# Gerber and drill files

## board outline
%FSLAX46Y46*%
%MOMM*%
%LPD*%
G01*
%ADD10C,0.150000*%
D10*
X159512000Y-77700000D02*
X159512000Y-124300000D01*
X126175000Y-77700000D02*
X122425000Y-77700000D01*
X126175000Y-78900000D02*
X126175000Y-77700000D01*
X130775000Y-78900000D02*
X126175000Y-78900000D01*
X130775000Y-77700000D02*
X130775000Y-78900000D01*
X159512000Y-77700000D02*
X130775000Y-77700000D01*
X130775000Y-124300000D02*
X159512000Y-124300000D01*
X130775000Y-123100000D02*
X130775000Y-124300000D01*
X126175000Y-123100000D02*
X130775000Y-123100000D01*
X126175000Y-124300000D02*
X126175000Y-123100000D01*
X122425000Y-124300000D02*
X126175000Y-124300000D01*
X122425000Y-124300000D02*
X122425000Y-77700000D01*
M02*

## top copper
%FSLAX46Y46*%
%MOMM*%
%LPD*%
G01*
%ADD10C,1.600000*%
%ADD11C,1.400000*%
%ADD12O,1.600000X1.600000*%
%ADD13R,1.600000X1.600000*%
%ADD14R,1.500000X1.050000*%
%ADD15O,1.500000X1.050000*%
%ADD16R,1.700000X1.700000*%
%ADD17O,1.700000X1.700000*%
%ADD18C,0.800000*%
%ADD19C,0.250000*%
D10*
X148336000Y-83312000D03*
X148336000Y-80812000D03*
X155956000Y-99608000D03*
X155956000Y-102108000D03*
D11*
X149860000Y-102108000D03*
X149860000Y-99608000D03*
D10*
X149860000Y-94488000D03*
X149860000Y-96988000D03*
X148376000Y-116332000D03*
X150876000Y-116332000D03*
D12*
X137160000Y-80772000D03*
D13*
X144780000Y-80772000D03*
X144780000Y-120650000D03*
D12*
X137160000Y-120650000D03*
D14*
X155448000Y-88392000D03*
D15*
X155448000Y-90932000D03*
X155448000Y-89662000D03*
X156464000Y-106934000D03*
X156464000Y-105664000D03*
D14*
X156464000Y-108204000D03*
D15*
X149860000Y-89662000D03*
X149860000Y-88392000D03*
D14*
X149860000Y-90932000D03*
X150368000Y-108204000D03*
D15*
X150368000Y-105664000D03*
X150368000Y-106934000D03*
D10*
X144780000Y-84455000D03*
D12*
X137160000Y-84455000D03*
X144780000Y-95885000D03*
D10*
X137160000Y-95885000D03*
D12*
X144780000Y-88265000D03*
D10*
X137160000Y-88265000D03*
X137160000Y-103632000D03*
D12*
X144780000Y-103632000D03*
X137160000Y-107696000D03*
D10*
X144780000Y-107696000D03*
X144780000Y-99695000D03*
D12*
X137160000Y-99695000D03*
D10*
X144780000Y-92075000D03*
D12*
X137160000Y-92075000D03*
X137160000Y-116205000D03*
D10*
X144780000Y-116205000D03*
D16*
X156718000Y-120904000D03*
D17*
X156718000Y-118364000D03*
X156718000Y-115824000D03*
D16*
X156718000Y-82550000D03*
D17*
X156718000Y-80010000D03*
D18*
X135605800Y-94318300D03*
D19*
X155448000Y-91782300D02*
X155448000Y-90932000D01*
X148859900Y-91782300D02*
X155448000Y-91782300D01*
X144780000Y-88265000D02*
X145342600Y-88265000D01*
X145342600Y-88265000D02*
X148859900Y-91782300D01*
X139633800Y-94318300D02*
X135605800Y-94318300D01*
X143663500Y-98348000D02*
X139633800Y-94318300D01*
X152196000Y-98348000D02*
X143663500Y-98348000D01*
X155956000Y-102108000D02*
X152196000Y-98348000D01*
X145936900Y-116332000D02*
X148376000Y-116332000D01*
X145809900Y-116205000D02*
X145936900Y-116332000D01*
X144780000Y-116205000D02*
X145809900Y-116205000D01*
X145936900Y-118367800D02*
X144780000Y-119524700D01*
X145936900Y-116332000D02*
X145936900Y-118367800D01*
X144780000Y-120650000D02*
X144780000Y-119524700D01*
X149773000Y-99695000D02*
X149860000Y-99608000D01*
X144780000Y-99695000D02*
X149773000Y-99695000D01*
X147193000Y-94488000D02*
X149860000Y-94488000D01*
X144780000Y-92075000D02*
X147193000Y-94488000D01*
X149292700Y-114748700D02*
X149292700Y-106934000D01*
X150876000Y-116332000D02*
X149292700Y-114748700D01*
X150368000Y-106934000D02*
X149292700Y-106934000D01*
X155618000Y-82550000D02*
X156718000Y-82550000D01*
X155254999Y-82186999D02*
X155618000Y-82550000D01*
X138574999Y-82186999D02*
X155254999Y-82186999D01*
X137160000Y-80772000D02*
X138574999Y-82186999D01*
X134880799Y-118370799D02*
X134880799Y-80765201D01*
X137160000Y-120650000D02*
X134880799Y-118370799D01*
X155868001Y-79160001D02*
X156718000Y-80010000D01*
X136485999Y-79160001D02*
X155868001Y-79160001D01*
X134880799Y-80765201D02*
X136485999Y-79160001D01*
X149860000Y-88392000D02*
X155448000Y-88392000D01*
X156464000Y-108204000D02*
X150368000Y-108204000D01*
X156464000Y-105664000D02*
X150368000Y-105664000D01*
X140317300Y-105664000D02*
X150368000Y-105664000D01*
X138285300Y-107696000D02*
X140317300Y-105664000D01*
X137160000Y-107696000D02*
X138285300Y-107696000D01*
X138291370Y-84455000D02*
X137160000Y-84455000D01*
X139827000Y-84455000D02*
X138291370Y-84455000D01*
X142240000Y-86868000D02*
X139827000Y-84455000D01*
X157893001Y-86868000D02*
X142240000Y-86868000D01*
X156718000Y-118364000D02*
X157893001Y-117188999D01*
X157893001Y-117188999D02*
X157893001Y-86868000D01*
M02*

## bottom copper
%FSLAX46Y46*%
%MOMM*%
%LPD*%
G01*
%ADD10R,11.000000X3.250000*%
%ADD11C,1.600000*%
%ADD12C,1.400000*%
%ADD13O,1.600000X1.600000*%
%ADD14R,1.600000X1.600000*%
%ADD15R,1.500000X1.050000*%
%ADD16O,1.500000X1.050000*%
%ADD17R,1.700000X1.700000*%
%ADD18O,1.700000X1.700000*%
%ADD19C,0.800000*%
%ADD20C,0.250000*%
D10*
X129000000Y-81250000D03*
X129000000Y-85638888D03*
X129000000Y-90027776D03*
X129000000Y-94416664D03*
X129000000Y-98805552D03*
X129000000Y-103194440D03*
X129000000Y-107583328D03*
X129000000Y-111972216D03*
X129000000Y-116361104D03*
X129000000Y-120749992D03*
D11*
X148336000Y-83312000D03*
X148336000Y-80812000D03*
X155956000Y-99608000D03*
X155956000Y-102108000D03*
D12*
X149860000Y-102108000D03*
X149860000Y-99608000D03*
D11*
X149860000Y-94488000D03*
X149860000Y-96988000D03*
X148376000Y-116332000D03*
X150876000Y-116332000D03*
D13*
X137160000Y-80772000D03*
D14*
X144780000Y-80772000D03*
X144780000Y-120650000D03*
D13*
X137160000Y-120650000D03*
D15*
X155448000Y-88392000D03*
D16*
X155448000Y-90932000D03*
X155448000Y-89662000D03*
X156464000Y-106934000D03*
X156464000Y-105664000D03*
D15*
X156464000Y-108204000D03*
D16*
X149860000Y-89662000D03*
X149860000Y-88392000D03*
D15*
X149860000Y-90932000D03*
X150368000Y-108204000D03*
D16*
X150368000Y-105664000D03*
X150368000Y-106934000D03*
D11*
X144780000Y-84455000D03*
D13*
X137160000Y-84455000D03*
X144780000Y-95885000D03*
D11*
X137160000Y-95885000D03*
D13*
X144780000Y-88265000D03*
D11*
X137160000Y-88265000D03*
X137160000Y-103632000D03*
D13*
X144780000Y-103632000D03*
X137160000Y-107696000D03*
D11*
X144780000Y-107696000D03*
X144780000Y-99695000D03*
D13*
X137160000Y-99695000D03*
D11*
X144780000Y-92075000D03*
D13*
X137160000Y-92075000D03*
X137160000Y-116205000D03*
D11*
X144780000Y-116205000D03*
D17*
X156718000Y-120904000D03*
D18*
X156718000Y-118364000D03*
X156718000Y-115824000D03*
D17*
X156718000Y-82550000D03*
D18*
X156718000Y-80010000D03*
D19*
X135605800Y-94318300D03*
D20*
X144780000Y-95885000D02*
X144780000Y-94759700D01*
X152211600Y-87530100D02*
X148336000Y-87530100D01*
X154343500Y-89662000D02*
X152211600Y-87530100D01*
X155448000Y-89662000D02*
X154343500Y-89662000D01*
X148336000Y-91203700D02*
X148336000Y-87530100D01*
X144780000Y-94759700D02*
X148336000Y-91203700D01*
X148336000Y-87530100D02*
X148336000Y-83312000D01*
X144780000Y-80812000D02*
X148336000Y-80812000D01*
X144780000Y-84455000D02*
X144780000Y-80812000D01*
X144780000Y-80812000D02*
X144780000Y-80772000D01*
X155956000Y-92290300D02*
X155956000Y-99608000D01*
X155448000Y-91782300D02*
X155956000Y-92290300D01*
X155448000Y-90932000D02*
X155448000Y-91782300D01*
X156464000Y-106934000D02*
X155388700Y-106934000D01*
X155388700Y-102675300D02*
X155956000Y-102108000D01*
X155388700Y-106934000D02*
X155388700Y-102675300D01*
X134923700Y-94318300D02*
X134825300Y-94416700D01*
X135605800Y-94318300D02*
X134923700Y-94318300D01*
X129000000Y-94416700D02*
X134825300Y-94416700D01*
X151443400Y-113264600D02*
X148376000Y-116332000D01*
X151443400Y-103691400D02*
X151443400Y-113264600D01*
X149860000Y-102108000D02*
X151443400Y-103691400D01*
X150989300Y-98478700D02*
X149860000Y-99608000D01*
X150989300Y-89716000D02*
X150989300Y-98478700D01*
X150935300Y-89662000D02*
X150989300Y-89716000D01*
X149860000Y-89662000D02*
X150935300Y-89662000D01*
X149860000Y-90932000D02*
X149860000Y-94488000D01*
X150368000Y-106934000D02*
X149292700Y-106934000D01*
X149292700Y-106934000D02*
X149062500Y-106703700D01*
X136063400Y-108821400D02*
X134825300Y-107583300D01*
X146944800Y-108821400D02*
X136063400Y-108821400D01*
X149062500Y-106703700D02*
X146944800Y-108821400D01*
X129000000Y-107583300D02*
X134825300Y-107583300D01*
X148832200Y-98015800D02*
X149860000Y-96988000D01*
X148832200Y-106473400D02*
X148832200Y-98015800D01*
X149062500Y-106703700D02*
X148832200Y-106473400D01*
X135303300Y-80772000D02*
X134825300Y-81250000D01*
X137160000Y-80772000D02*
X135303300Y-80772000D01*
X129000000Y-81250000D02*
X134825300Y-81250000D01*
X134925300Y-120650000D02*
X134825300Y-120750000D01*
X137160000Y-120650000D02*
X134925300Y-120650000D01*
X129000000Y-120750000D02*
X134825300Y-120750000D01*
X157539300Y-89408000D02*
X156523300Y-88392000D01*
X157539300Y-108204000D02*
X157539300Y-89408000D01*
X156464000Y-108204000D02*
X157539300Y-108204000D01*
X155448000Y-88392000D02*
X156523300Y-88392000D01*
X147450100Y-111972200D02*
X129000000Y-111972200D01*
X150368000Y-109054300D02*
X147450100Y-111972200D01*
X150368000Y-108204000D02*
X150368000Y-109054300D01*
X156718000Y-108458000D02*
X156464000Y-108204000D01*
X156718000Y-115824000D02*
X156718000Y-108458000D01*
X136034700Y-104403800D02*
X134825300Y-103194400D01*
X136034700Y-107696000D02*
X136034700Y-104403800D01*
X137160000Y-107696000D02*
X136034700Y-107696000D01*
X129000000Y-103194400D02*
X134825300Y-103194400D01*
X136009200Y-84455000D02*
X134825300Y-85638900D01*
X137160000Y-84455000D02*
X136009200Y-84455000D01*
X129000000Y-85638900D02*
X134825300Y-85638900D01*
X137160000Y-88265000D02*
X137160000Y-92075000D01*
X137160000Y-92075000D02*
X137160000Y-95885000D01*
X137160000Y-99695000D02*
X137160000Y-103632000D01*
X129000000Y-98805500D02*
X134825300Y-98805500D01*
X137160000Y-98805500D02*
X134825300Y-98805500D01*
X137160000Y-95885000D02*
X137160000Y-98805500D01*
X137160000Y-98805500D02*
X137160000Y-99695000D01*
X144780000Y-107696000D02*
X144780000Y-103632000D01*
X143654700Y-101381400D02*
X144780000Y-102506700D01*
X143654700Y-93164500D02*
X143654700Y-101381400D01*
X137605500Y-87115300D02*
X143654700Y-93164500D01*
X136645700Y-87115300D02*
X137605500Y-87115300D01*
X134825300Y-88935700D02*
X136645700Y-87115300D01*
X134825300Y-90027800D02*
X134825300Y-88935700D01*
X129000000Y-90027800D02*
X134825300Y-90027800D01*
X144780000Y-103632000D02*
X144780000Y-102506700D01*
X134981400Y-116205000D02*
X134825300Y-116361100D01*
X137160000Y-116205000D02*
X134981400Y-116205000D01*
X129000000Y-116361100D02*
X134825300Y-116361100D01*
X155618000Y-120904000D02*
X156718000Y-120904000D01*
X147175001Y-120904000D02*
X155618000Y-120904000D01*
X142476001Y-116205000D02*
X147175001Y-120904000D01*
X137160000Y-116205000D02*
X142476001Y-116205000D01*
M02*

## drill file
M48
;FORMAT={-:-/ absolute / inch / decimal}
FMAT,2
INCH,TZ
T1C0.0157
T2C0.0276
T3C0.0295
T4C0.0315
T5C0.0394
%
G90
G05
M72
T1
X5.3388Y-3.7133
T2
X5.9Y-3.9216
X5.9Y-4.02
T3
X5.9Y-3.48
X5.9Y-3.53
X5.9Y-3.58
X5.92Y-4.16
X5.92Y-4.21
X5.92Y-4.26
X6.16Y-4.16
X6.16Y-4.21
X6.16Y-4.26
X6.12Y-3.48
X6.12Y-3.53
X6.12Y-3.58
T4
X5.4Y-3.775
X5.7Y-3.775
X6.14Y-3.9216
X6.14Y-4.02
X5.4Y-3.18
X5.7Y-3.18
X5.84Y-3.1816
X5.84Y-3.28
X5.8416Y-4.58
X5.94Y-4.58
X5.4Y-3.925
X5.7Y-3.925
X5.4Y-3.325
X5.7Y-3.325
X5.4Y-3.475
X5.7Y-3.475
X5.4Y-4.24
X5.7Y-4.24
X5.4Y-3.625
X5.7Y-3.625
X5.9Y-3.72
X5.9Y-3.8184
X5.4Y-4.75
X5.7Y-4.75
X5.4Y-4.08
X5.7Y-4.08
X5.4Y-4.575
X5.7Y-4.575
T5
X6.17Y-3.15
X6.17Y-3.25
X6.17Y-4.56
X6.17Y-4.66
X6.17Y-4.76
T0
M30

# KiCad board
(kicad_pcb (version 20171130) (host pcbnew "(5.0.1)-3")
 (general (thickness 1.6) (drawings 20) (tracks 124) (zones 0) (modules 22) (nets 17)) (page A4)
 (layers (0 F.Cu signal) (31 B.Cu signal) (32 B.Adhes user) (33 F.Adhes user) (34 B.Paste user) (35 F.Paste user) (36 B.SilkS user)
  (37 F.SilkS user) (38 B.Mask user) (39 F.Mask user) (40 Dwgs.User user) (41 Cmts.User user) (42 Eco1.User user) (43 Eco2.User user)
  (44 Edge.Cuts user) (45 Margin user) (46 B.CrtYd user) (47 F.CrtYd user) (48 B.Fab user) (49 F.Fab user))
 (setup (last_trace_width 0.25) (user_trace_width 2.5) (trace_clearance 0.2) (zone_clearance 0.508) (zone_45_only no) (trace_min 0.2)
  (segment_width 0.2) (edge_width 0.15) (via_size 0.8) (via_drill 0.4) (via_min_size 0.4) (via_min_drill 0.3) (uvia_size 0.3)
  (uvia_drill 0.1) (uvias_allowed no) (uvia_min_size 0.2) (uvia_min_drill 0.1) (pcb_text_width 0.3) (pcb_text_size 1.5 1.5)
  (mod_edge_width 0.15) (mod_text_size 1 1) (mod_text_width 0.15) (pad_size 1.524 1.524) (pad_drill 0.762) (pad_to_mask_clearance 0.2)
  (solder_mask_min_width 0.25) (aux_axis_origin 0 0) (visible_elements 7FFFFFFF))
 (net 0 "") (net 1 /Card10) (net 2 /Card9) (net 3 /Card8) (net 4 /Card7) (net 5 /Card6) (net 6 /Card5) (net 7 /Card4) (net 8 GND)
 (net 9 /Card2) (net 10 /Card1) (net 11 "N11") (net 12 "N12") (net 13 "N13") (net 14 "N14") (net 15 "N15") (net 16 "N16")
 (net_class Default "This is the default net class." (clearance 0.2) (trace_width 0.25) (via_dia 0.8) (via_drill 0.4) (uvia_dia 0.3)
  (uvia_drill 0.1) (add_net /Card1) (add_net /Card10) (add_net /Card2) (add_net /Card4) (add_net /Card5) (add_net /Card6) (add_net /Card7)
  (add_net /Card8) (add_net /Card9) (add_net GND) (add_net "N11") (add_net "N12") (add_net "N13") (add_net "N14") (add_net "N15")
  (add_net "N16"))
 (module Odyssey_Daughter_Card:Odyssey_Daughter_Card (layer F.Cu) (at 129 101)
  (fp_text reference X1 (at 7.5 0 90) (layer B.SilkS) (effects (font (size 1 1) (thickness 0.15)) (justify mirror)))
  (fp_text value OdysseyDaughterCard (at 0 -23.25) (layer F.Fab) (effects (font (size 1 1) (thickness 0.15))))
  (pad 10 smd rect (at 0 -19.75) (size 11 3.25) (layers B.Cu B.Mask) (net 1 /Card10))
  (pad 9 smd rect (at 0 -15.361112) (size 11 3.25) (layers B.Cu B.Mask) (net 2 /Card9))
  (pad 8 smd rect (at 0 -10.972224) (size 11 3.25) (layers B.Cu B.Mask) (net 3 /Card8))
  (pad 7 smd rect (at 0 -6.583336) (size 11 3.25) (layers B.Cu B.Mask) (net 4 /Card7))
  (pad 6 smd rect (at 0 -2.194448) (size 11 3.25) (layers B.Cu B.Mask) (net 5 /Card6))
  (pad 5 smd rect (at 0 2.19444) (size 11 3.25) (layers B.Cu B.Mask) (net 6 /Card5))
  (pad 4 smd rect (at 0 6.583328) (size 11 3.25) (layers B.Cu B.Mask) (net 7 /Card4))
  (pad 3 smd rect (at 0 10.972216) (size 11 3.25) (layers B.Cu B.Mask) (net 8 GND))
  (pad 2 smd rect (at 0 15.361104) (size 11 3.25) (layers B.Cu B.Mask) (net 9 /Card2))
  (pad 1 smd rect (at 0 19.749992) (size 11 3.25) (layers B.Cu B.Mask) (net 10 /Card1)))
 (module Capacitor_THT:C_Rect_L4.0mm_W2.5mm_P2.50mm (layer F.Cu) (at 148.336 83.312 90)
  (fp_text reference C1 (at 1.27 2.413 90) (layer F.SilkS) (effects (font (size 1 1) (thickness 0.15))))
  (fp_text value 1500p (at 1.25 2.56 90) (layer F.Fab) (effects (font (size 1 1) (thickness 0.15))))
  (pad 1 thru_hole circle (at 0 0 90) (size 1.6 1.6) (drill 0.8) (layers *.Cu *.Mask) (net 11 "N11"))
  (pad 2 thru_hole circle (at 2.5 0 90) (size 1.6 1.6) (drill 0.8) (layers *.Cu *.Mask) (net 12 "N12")))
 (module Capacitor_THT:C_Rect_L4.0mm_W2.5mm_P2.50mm (layer F.Cu) (at 155.956 102.108 90)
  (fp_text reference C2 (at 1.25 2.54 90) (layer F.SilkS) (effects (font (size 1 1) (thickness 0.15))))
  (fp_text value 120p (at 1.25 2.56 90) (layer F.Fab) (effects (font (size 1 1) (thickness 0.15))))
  (pad 2 thru_hole circle (at 2.5 0 90) (size 1.6 1.6) (drill 0.8) (layers *.Cu *.Mask) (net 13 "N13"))
  (pad 1 thru_hole circle (at 0 0 90) (size 1.6 1.6) (drill 0.8) (layers *.Cu *.Mask) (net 4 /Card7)))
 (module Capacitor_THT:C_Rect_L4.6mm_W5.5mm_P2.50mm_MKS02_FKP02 (layer F.Cu) (at 149.86 102.108 90)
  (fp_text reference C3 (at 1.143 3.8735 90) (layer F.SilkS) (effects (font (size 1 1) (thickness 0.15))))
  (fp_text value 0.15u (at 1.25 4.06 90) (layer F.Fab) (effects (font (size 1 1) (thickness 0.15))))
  (pad 1 thru_hole circle (at 0 0 90) (size 1.4 1.4) (drill 0.7) (layers *.Cu *.Mask) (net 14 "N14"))
  (pad 2 thru_hole circle (at 2.5 0 90) (size 1.4 1.4) (drill 0.7) (layers *.Cu *.Mask) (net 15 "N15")))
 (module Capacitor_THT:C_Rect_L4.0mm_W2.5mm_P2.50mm (layer F.Cu) (at 149.86 94.488 270)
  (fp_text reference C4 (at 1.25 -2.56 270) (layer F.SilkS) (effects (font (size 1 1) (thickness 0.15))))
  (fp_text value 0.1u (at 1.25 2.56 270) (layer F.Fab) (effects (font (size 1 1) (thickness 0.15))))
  (pad 1 thru_hole circle (at 0 0 270) (size 1.6 1.6) (drill 0.8) (layers *.Cu *.Mask) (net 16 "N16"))
  (pad 2 thru_hole circle (at 2.5 0 270) (size 1.6 1.6) (drill 0.8) (layers *.Cu *.Mask) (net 7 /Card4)))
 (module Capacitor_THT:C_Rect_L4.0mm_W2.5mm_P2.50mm (layer F.Cu) (at 150.876 116.332 180)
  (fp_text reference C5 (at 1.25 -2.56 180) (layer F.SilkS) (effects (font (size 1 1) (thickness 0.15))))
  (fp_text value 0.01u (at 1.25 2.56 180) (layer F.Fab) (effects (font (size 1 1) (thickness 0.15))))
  (pad 2 thru_hole circle (at 2.5 0 180) (size 1.6 1.6) (drill 0.8) (layers *.Cu *.Mask) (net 14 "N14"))
  (pad 1 thru_hole circle (at 0 0 180) (size 1.6 1.6) (drill 0.8) (layers *.Cu *.Mask) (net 7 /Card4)))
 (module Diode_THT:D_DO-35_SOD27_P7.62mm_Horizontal (layer F.Cu) (at 144.78 80.772 180)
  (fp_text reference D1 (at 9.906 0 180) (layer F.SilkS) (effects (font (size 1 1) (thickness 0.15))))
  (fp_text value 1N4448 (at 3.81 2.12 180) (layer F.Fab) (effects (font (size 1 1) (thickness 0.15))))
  (pad 2 thru_hole oval (at 7.62 0 180) (size 1.6 1.6) (drill 0.8) (layers *.Cu *.Mask) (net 1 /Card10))
  (pad 1 thru_hole rect (at 0 0 180) (size 1.6 1.6) (drill 0.8) (layers *.Cu *.Mask) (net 12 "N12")))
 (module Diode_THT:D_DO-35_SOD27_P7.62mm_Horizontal (layer F.Cu) (at 144.78 120.65 180)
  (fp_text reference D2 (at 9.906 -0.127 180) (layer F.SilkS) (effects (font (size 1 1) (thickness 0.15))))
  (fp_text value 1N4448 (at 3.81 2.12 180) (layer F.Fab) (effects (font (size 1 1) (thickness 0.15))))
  (pad 1 thru_hole rect (at 0 0 180) (size 1.6 1.6) (drill 0.8) (layers *.Cu *.Mask) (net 14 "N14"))
  (pad 2 thru_hole oval (at 7.62 0 180) (size 1.6 1.6) (drill 0.8) (layers *.Cu *.Mask) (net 10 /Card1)))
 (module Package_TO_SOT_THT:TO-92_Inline (layer F.Cu) (at 155.448 88.392 270)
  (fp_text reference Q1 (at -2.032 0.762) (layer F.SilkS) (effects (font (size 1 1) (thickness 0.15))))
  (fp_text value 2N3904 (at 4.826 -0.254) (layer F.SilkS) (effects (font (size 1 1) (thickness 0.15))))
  (pad 1 thru_hole rect (at 0 0 270) (size 1.05 1.5) (drill 0.75) (layers *.Cu *.Mask) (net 8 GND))
  (pad 3 thru_hole oval (at 2.54 0 270) (size 1.05 1.5) (drill 0.75) (layers *.Cu *.Mask) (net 13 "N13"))
  (pad 2 thru_hole oval (at 1.27 0 270) (size 1.05 1.5) (drill 0.75) (layers *.Cu *.Mask) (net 11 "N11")))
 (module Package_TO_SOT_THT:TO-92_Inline (layer F.Cu) (at 156.464 108.204 90)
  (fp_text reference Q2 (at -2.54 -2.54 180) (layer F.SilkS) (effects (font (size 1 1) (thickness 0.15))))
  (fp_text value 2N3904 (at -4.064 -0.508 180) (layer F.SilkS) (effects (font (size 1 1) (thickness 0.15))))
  (pad 2 thru_hole oval (at 1.27 0 90) (size 1.05 1.5) (drill 0.75) (layers *.Cu *.Mask) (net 4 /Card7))
  (pad 3 thru_hole oval (at 2.54 0 90) (size 1.05 1.5) (drill 0.75) (layers *.Cu *.Mask) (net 6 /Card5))
  (pad 1 thru_hole rect (at 0 0 90) (size 1.05 1.5) (drill 0.75) (layers *.Cu *.Mask) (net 8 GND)))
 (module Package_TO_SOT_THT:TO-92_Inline (layer F.Cu) (at 149.86 90.932 90)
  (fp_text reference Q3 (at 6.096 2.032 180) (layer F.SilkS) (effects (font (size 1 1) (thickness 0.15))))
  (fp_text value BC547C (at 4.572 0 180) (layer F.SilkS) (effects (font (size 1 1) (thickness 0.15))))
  (pad 2 thru_hole oval (at 1.27 0 90) (size 1.05 1.5) (drill 0.75) (layers *.Cu *.Mask) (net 15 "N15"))
  (pad 3 thru_hole oval (at 2.54 0 90) (size 1.05 1.5) (drill 0.75) (layers *.Cu *.Mask) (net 8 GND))
  (pad 1 thru_hole rect (at 0 0 90) (size 1.05 1.5) (drill 0.75) (layers *.Cu *.Mask) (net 16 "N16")))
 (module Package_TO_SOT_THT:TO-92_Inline (layer F.Cu) (at 150.368 108.204 90)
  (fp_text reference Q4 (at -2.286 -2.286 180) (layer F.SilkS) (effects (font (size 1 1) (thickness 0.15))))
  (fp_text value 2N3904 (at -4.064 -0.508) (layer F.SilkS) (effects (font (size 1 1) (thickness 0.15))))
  (pad 1 thru_hole rect (at 0 0 90) (size 1.05 1.5) (drill 0.75) (layers *.Cu *.Mask) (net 8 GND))
  (pad 3 thru_hole oval (at 2.54 0 90) (size 1.05 1.5) (drill 0.75) (layers *.Cu *.Mask) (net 6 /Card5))
  (pad 2 thru_hole oval (at 1.27 0 90) (size 1.05 1.5) (drill 0.75) (layers *.Cu *.Mask) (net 7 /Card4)))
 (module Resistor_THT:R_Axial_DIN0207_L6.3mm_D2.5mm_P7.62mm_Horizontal (layer F.Cu) (at 144.78 84.455 180)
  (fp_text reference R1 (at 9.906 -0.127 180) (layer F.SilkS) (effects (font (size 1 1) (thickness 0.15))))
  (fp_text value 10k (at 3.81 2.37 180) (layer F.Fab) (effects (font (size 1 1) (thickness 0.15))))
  (pad 1 thru_hole circle (at 0 0 180) (size 1.6 1.6) (drill 0.8) (layers *.Cu *.Mask) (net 12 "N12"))
  (pad 2 thru_hole oval (at 7.62 0 180) (size 1.6 1.6) (drill 0.8) (layers *.Cu *.Mask) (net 2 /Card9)))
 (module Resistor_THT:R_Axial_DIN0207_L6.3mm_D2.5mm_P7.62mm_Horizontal (layer F.Cu) (at 137.16 95.885)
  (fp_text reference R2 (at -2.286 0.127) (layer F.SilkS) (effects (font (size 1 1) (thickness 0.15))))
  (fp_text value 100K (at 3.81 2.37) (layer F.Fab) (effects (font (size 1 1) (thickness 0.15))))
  (pad 2 thru_hole oval (at 7.62 0) (size 1.6 1.6) (drill 0.8) (layers *.Cu *.Mask) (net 11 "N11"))
  (pad 1 thru_hole circle (at 0 0) (size 1.6 1.6) (drill 0.8) (layers *.Cu *.Mask) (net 5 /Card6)))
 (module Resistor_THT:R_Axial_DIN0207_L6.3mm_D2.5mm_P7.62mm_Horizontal (layer F.Cu) (at 137.16 88.265)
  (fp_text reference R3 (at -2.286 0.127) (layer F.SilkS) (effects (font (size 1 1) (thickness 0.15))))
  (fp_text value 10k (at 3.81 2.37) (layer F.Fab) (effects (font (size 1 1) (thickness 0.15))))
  (pad 2 thru_hole oval (at 7.62 0) (size 1.6 1.6) (drill 0.8) (layers *.Cu *.Mask) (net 13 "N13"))
  (pad 1 thru_hole circle (at 0 0) (size 1.6 1.6) (drill 0.8) (layers *.Cu *.Mask) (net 5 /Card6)))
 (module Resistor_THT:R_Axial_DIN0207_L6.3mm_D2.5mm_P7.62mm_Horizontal (layer F.Cu) (at 137.16 103.632)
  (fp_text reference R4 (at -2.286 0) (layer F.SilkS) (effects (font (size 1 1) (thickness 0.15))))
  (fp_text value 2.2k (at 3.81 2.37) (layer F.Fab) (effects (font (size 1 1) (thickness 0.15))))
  (pad 1 thru_hole circle (at 0 0) (size 1.6 1.6) (drill 0.8) (layers *.Cu *.Mask) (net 5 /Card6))
  (pad 2 thru_hole oval (at 7.62 0) (size 1.6 1.6) (drill 0.8) (layers *.Cu *.Mask) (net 3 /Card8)))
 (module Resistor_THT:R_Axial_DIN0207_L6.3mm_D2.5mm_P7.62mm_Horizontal (layer F.Cu) (at 144.78 107.696 180)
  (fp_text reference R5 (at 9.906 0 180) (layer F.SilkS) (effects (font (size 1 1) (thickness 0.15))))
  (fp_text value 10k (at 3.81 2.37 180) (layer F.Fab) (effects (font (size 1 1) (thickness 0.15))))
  (pad 2 thru_hole oval (at 7.62 0 180) (size 1.6 1.6) (drill 0.8) (layers *.Cu *.Mask) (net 6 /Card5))
  (pad 1 thru_hole circle (at 0 0 180) (size 1.6 1.6) (drill 0.8) (layers *.Cu *.Mask) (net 3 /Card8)))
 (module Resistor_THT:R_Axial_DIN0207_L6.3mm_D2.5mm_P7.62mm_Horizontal (layer F.Cu) (at 144.78 99.695 180)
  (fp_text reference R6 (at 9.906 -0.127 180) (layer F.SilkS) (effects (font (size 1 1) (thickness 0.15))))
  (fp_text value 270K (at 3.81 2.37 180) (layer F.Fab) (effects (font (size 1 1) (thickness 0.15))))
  (pad 1 thru_hole circle (at 0 0 180) (size 1.6 1.6) (drill 0.8) (layers *.Cu *.Mask) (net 15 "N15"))
  (pad 2 thru_hole oval (at 7.62 0 180) (size 1.6 1.6) (drill 0.8) (layers *.Cu *.Mask) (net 5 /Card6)))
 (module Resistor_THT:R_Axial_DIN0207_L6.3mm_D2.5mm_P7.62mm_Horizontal (layer F.Cu) (at 144.78 92.075 180)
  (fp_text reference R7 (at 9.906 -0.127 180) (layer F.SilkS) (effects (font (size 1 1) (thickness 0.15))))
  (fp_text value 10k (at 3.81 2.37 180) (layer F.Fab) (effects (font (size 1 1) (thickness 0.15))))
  (pad 1 thru_hole circle (at 0 0 180) (size 1.6 1.6) (drill 0.8) (layers *.Cu *.Mask) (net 16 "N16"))
  (pad 2 thru_hole oval (at 7.62 0 180) (size 1.6 1.6) (drill 0.8) (layers *.Cu *.Mask) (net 5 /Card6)))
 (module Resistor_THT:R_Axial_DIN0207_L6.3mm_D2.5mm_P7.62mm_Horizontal (layer F.Cu) (at 144.78 116.205 180)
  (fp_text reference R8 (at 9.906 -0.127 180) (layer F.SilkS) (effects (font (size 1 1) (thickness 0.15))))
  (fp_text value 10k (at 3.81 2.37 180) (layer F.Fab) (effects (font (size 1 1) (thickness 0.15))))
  (pad 2 thru_hole oval (at 7.62 0 180) (size 1.6 1.6) (drill 0.8) (layers *.Cu *.Mask) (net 9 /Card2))
  (pad 1 thru_hole circle (at 0 0 180) (size 1.6 1.6) (drill 0.8) (layers *.Cu *.Mask) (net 14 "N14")))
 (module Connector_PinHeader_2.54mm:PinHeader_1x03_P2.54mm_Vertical (layer F.Cu) (at 156.718 120.904 180)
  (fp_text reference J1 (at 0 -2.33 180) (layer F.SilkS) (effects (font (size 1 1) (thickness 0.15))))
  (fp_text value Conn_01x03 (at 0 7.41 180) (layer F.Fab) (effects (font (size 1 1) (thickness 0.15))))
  (pad 1 thru_hole rect (at 0 0 180) (size 1.7 1.7) (drill 1) (layers *.Cu *.Mask) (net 9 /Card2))
  (pad 2 thru_hole oval (at 0 2.54 180) (size 1.7 1.7) (drill 1) (layers *.Cu *.Mask) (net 2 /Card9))
  (pad 3 thru_hole oval (at 0 5.08 180) (size 1.7 1.7) (drill 1) (layers *.Cu *.Mask) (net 8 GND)))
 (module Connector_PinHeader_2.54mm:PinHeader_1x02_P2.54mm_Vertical (layer F.Cu) (at 156.718 82.55 180)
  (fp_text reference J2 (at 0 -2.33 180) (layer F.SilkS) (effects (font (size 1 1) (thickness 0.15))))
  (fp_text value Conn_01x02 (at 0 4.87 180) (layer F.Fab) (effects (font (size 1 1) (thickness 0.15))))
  (pad 1 thru_hole rect (at 0 0 180) (size 1.7 1.7) (drill 1) (layers *.Cu *.Mask) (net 1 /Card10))
  (pad 2 thru_hole oval (at 0 2.54 180) (size 1.7 1.7) (drill 1) (layers *.Cu *.Mask) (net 10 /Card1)))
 (gr_line (start 159.512 77.7) (end 159.512 124.3) (layer Edge.Cuts) (width 0.15))
 (gr_line (start 126.175 77.7) (end 122.425 77.7) (layer Edge.Cuts) (width 0.15))
 (gr_line (start 126.175 78.9) (end 126.175 77.7) (layer Edge.Cuts) (width 0.15))
 (gr_line (start 130.775 78.9) (end 126.175 78.9) (layer Edge.Cuts) (width 0.15))
 (gr_line (start 130.775 77.7) (end 130.775 78.9) (layer Edge.Cuts) (width 0.15))
 (gr_line (start 159.512 77.7) (end 130.775 77.7) (layer Edge.Cuts) (width 0.15))
 (gr_line (start 130.775 124.3) (end 159.512 124.3) (layer Edge.Cuts) (width 0.15))
 (gr_line (start 130.775 123.1) (end 130.775 124.3) (layer Edge.Cuts) (width 0.15))
 (gr_line (start 126.175 123.1) (end 130.775 123.1) (layer Edge.Cuts) (width 0.15))
 (gr_line (start 126.175 124.3) (end 126.175 123.1) (layer Edge.Cuts) (width 0.15))
 (gr_line (start 122.425 124.3) (end 126.175 124.3) (layer Edge.Cuts) (width 0.15))
 (gr_line (start 122.425 124.3) (end 122.425 77.7) (layer Edge.Cuts) (width 0.15))
 (segment (start 144.78 95.885) (end 144.78 94.7597) (width 0.25) (layer B.Cu) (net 11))
 (segment (start 152.2116 87.5301) (end 148.336 87.5301) (width 0.25) (layer B.Cu) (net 11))
 (segment (start 154.3435 89.662) (end 152.2116 87.5301) (width 0.25) (layer B.Cu) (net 11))
 (segment (start 155.448 89.662) (end 154.3435 89.662) (width 0.25) (layer B.Cu) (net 11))
 (segment (start 148.336 91.2037) (end 148.336 87.5301) (width 0.25) (layer B.Cu) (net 11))
 (segment (start 144.78 94.7597) (end 148.336 91.2037) (width 0.25) (layer B.Cu) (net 11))
 (segment (start 148.336 87.5301) (end 148.336 83.312) (width 0.25) (layer B.Cu) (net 11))
 (segment (start 144.78 80.812) (end 148.336 80.812) (width 0.25) (layer B.Cu) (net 12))
 (segment (start 144.78 84.455) (end 144.78 80.812) (width 0.25) (layer B.Cu) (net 12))
 (segment (start 144.78 80.812) (end 144.78 80.772) (width 0.25) (layer B.Cu) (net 12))
 (segment (start 155.956 92.2903) (end 155.956 99.608) (width 0.25) (layer B.Cu) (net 13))
 (segment (start 155.448 91.7823) (end 155.956 92.2903) (width 0.25) (layer B.Cu) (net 13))
 (segment (start 155.448 90.932) (end 155.448 91.7823) (width 0.25) (layer B.Cu) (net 13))
 (segment (start 155.448 91.7823) (end 155.448 90.932) (width 0.25) (layer F.Cu) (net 13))
 (segment (start 148.8599 91.7823) (end 155.448 91.7823) (width 0.25) (layer F.Cu) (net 13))
 (segment (start 144.78 88.265) (end 145.3426 88.265) (width 0.25) (layer F.Cu) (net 13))
 (segment (start 145.3426 88.265) (end 148.8599 91.7823) (width 0.25) (layer F.Cu) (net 13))
 (via (at 135.6058 94.3183) (size 0.8) (layers F.Cu B.Cu) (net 4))
 (segment (start 156.464 106.934) (end 155.3887 106.934) (width 0.25) (layer B.Cu) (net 4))
 (segment (start 155.3887 102.6753) (end 155.956 102.108) (width 0.25) (layer B.Cu) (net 4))
 (segment (start 155.3887 106.934) (end 155.3887 102.6753) (width 0.25) (layer B.Cu) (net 4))
 (segment (start 139.6338 94.3183) (end 135.6058 94.3183) (width 0.25) (layer F.Cu) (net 4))
 (segment (start 143.6635 98.348) (end 139.6338 94.3183) (width 0.25) (layer F.Cu) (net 4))
 (segment (start 152.196 98.348) (end 143.6635 98.348) (width 0.25) (layer F.Cu) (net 4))
 (segment (start 155.956 102.108) (end 152.196 98.348) (width 0.25) (layer F.Cu) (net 4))
 (segment (start 134.9237 94.3183) (end 134.8253 94.4167) (width 0.25) (layer B.Cu) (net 4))
 (segment (start 135.6058 94.3183) (end 134.9237 94.3183) (width 0.25) (layer B.Cu) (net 4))
 (segment (start 129 94.4167) (end 134.8253 94.4167) (width 0.25) (layer B.Cu) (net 4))
 (segment (start 151.4434 113.2646) (end 148.376 116.332) (width 0.25) (layer B.Cu) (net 14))
 (segment (start 151.4434 103.6914) (end 151.4434 113.2646) (width 0.25) (layer B.Cu) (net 14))
 (segment (start 149.86 102.108) (end 151.4434 103.6914) (width 0.25) (layer B.Cu) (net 14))
 (segment (start 145.9369 116.332) (end 148.376 116.332) (width 0.25) (layer F.Cu) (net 14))
 (segment (start 145.8099 116.205) (end 145.9369 116.332) (width 0.25) (layer F.Cu) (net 14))
 (segment (start 144.78 116.205) (end 145.8099 116.205) (width 0.25) (layer F.Cu) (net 14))
 (segment (start 145.9369 118.3678) (end 144.78 119.5247) (width 0.25) (layer F.Cu) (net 14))
 (segment (start 145.9369 116.332) (end 145.9369 118.3678) (width 0.25) (layer F.Cu) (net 14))
 (segment (start 144.78 120.65) (end 144.78 119.5247) (width 0.25) (layer F.Cu) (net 14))
 (segment (start 150.9893 98.4787) (end 149.86 99.608) (width 0.25) (layer B.Cu) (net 15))
 (segment (start 150.9893 89.716) (end 150.9893 98.4787) (width 0.25) (layer B.Cu) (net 15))
 (segment (start 150.9353 89.662) (end 150.9893 89.716) (width 0.25) (layer B.Cu) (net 15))
 (segment (start 149.86 89.662) (end 150.9353 89.662) (width 0.25) (layer B.Cu) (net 15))
 (segment (start 149.773 99.695) (end 149.86 99.608) (width 0.25) (layer F.Cu) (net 15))
 (segment (start 144.78 99.695) (end 149.773 99.695) (width 0.25) (layer F.Cu) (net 15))
 (segment (start 147.193 94.488) (end 149.86 94.488) (width 0.25) (layer F.Cu) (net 16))
 (segment (start 144.78 92.075) (end 147.193 94.488) (width 0.25) (layer F.Cu) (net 16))
 (segment (start 149.86 90.932) (end 149.86 94.488) (width 0.25) (layer B.Cu) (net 16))
 (segment (start 149.2927 114.7487) (end 149.2927 106.934) (width 0.25) (layer F.Cu) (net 7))
 (segment (start 150.876 116.332) (end 149.2927 114.7487) (width 0.25) (layer F.Cu) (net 7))
 (segment (start 150.368 106.934) (end 149.2927 106.934) (width 0.25) (layer F.Cu) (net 7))
 (segment (start 150.368 106.934) (end 149.2927 106.934) (width 0.25) (layer B.Cu) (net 7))
 (segment (start 149.2927 106.934) (end 149.0625 106.7037) (width 0.25) (layer B.Cu) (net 7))
 (segment (start 136.0634 108.8214) (end 134.8253 107.5833) (width 0.25) (layer B.Cu) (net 7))
 (segment (start 146.9448 108.8214) (end 136.0634 108.8214) (width 0.25) (layer B.Cu) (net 7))
 (segment (start 149.0625 106.7037) (end 146.9448 108.8214) (width 0.25) (layer B.Cu) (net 7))
 (segment (start 129 107.5833) (end 134.8253 107.5833) (width 0.25) (layer B.Cu) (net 7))
 (segment (start 148.8322 98.0158) (end 149.86 96.988) (width 0.25) (layer B.Cu) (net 7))
 (segment (start 148.8322 106.4734) (end 148.8322 98.0158) (width 0.25) (layer B.Cu) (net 7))
 (segment (start 149.0625 106.7037) (end 148.8322 106.4734) (width 0.25) (layer B.Cu) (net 7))
 (segment (start 135.3033 80.772) (end 134.8253 81.25) (width 0.25) (layer B.Cu) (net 1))
 (segment (start 137.16 80.772) (end 135.3033 80.772) (width 0.25) (layer B.Cu) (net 1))
 (segment (start 129 81.25) (end 134.8253 81.25) (width 0.25) (layer B.Cu) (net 1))
 (segment (start 155.618 82.55) (end 156.718 82.55) (width 0.25) (layer F.Cu) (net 1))
 (segment (start 155.254999 82.186999) (end 155.618 82.55) (width 0.25) (layer F.Cu) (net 1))
 (segment (start 138.574999 82.186999) (end 155.254999 82.186999) (width 0.25) (layer F.Cu) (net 1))
 (segment (start 137.16 80.772) (end 138.574999 82.186999) (width 0.25) (layer F.Cu) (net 1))
 (segment (start 134.9253 120.65) (end 134.8253 120.75) (width 0.25) (layer B.Cu) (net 10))
 (segment (start 137.16 120.65) (end 134.9253 120.65) (width 0.25) (layer B.Cu) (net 10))
 (segment (start 129 120.75) (end 134.8253 120.75) (width 0.25) (layer B.Cu) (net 10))
 (segment (start 134.880799 118.370799) (end 134.880799 80.765201) (width 0.25) (layer F.Cu) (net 10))
 (segment (start 137.16 120.65) (end 134.880799 118.370799) (width 0.25) (layer F.Cu) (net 10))
 (segment (start 155.868001 79.160001) (end 156.718 80.01) (width 0.25) (layer F.Cu) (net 10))
 (segment (start 136.485999 79.160001) (end 155.868001 79.160001) (width 0.25) (layer F.Cu) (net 10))
 (segment (start 134.880799 80.765201) (end 136.485999 79.160001) (width 0.25) (layer F.Cu) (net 10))
 (segment (start 149.86 88.392) (end 155.448 88.392) (width 0.25) (layer F.Cu) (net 8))
 (segment (start 156.464 108.204) (end 150.368 108.204) (width 0.25) (layer F.Cu) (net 8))
 (segment (start 157.5393 89.408) (end 156.5233 88.392) (width 0.25) (layer B.Cu) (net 8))
 (segment (start 157.5393 108.204) (end 157.5393 89.408) (width 0.25) (layer B.Cu) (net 8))
 (segment (start 156.464 108.204) (end 157.5393 108.204) (width 0.25) (layer B.Cu) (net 8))
 (segment (start 155.448 88.392) (end 156.5233 88.392) (width 0.25) (layer B.Cu) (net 8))
 (segment (start 147.4501 111.9722) (end 129 111.9722) (width 0.25) (layer B.Cu) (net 8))
 (segment (start 150.368 109.0543) (end 147.4501 111.9722) (width 0.25) (layer B.Cu) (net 8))
 (segment (start 150.368 108.204) (end 150.368 109.0543) (width 0.25) (layer B.Cu) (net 8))
 (segment (start 156.718 108.458) (end 156.464 108.204) (width 0.25) (layer B.Cu) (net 8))
 (segment (start 156.718 115.824) (end 156.718 108.458) (width 0.25) (layer B.Cu) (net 8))
 (segment (start 156.464 105.664) (end 150.368 105.664) (width 0.25) (layer F.Cu) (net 6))
 (segment (start 136.0347 104.4038) (end 134.8253 103.1944) (width 0.25) (layer B.Cu) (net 6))
 (segment (start 136.0347 107.696) (end 136.0347 104.4038) (width 0.25) (layer B.Cu) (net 6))
 (segment (start 137.16 107.696) (end 136.0347 107.696) (width 0.25) (layer B.Cu) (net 6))
 (segment (start 129 103.1944) (end 134.8253 103.1944) (width 0.25) (layer B.Cu) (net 6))
 (segment (start 140.3173 105.664) (end 150.368 105.664) (width 0.25) (layer F.Cu) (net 6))
 (segment (start 138.2853 107.696) (end 140.3173 105.664) (width 0.25) (layer F.Cu) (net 6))
 (segment (start 137.16 107.696) (end 138.2853 107.696) (width 0.25) (layer F.Cu) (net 6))
 (segment (start 136.0092 84.455) (end 134.8253 85.6389) (width 0.25) (layer B.Cu) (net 2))
 (segment (start 137.16 84.455) (end 136.0092 84.455) (width 0.25) (layer B.Cu) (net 2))
 (segment (start 129 85.6389) (end 134.8253 85.6389) (width 0.25) (layer B.Cu) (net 2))
 (segment (start 138.29137 84.455) (end 137.16 84.455) (width 0.25) (layer F.Cu) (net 2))
 (segment (start 139.827 84.455) (end 138.29137 84.455) (width 0.25) (layer F.Cu) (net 2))
 (segment (start 142.24 86.868) (end 139.827 84.455) (width 0.25) (layer F.Cu) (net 2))
 (segment (start 157.893001 86.868) (end 142.24 86.868) (width 0.25) (layer F.Cu) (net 2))
 (segment (start 156.718 118.364) (end 157.893001 117.188999) (width 0.25) (layer F.Cu) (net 2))
 (segment (start 157.893001 117.188999) (end 157.893001 86.868) (width 0.25) (layer F.Cu) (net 2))
 (segment (start 137.16 88.265) (end 137.16 92.075) (width 0.25) (layer B.Cu) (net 5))
 (segment (start 137.16 92.075) (end 137.16 95.885) (width 0.25) (layer B.Cu) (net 5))
 (segment (start 137.16 99.695) (end 137.16 103.632) (width 0.25) (layer B.Cu) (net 5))
 (segment (start 129 98.8055) (end 134.8253 98.8055) (width 0.25) (layer B.Cu) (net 5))
 (segment (start 137.16 98.8055) (end 134.8253 98.8055) (width 0.25) (layer B.Cu) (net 5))
 (segment (start 137.16 95.885) (end 137.16 98.8055) (width 0.25) (layer B.Cu) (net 5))
 (segment (start 137.16 98.8055) (end 137.16 99.695) (width 0.25) (layer B.Cu) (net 5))
 (segment (start 144.78 107.696) (end 144.78 103.632) (width 0.25) (layer B.Cu) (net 3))
 (segment (start 143.6547 101.3814) (end 144.78 102.5067) (width 0.25) (layer B.Cu) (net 3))
 (segment (start 143.6547 93.1645) (end 143.6547 101.3814) (width 0.25) (layer B.Cu) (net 3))
 (segment (start 137.6055 87.1153) (end 143.6547 93.1645) (width 0.25) (layer B.Cu) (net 3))
 (segment (start 136.6457 87.1153) (end 137.6055 87.1153) (width 0.25) (layer B.Cu) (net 3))
 (segment (start 134.8253 88.9357) (end 136.6457 87.1153) (width 0.25) (layer B.Cu) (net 3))
 (segment (start 134.8253 90.0278) (end 134.8253 88.9357) (width 0.25) (layer B.Cu) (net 3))
 (segment (start 129 90.0278) (end 134.8253 90.0278) (width 0.25) (layer B.Cu) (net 3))
 (segment (start 144.78 103.632) (end 144.78 102.5067) (width 0.25) (layer B.Cu) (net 3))
 (segment (start 134.9814 116.205) (end 134.8253 116.3611) (width 0.25) (layer B.Cu) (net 9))
 (segment (start 137.16 116.205) (end 134.9814 116.205) (width 0.25) (layer B.Cu) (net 9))
 (segment (start 129 116.3611) (end 134.8253 116.3611) (width 0.25) (layer B.Cu) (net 9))
 (segment (start 155.618 120.904) (end 156.718 120.904) (width 0.25) (layer B.Cu) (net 9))
 (segment (start 147.175001 120.904) (end 155.618 120.904) (width 0.25) (layer B.Cu) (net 9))
 (segment (start 142.476001 116.205) (end 147.175001 120.904) (width 0.25) (layer B.Cu) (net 9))
 (segment (start 137.16 116.205) (end 142.476001 116.205) (width 0.25) (layer B.Cu) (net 9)))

